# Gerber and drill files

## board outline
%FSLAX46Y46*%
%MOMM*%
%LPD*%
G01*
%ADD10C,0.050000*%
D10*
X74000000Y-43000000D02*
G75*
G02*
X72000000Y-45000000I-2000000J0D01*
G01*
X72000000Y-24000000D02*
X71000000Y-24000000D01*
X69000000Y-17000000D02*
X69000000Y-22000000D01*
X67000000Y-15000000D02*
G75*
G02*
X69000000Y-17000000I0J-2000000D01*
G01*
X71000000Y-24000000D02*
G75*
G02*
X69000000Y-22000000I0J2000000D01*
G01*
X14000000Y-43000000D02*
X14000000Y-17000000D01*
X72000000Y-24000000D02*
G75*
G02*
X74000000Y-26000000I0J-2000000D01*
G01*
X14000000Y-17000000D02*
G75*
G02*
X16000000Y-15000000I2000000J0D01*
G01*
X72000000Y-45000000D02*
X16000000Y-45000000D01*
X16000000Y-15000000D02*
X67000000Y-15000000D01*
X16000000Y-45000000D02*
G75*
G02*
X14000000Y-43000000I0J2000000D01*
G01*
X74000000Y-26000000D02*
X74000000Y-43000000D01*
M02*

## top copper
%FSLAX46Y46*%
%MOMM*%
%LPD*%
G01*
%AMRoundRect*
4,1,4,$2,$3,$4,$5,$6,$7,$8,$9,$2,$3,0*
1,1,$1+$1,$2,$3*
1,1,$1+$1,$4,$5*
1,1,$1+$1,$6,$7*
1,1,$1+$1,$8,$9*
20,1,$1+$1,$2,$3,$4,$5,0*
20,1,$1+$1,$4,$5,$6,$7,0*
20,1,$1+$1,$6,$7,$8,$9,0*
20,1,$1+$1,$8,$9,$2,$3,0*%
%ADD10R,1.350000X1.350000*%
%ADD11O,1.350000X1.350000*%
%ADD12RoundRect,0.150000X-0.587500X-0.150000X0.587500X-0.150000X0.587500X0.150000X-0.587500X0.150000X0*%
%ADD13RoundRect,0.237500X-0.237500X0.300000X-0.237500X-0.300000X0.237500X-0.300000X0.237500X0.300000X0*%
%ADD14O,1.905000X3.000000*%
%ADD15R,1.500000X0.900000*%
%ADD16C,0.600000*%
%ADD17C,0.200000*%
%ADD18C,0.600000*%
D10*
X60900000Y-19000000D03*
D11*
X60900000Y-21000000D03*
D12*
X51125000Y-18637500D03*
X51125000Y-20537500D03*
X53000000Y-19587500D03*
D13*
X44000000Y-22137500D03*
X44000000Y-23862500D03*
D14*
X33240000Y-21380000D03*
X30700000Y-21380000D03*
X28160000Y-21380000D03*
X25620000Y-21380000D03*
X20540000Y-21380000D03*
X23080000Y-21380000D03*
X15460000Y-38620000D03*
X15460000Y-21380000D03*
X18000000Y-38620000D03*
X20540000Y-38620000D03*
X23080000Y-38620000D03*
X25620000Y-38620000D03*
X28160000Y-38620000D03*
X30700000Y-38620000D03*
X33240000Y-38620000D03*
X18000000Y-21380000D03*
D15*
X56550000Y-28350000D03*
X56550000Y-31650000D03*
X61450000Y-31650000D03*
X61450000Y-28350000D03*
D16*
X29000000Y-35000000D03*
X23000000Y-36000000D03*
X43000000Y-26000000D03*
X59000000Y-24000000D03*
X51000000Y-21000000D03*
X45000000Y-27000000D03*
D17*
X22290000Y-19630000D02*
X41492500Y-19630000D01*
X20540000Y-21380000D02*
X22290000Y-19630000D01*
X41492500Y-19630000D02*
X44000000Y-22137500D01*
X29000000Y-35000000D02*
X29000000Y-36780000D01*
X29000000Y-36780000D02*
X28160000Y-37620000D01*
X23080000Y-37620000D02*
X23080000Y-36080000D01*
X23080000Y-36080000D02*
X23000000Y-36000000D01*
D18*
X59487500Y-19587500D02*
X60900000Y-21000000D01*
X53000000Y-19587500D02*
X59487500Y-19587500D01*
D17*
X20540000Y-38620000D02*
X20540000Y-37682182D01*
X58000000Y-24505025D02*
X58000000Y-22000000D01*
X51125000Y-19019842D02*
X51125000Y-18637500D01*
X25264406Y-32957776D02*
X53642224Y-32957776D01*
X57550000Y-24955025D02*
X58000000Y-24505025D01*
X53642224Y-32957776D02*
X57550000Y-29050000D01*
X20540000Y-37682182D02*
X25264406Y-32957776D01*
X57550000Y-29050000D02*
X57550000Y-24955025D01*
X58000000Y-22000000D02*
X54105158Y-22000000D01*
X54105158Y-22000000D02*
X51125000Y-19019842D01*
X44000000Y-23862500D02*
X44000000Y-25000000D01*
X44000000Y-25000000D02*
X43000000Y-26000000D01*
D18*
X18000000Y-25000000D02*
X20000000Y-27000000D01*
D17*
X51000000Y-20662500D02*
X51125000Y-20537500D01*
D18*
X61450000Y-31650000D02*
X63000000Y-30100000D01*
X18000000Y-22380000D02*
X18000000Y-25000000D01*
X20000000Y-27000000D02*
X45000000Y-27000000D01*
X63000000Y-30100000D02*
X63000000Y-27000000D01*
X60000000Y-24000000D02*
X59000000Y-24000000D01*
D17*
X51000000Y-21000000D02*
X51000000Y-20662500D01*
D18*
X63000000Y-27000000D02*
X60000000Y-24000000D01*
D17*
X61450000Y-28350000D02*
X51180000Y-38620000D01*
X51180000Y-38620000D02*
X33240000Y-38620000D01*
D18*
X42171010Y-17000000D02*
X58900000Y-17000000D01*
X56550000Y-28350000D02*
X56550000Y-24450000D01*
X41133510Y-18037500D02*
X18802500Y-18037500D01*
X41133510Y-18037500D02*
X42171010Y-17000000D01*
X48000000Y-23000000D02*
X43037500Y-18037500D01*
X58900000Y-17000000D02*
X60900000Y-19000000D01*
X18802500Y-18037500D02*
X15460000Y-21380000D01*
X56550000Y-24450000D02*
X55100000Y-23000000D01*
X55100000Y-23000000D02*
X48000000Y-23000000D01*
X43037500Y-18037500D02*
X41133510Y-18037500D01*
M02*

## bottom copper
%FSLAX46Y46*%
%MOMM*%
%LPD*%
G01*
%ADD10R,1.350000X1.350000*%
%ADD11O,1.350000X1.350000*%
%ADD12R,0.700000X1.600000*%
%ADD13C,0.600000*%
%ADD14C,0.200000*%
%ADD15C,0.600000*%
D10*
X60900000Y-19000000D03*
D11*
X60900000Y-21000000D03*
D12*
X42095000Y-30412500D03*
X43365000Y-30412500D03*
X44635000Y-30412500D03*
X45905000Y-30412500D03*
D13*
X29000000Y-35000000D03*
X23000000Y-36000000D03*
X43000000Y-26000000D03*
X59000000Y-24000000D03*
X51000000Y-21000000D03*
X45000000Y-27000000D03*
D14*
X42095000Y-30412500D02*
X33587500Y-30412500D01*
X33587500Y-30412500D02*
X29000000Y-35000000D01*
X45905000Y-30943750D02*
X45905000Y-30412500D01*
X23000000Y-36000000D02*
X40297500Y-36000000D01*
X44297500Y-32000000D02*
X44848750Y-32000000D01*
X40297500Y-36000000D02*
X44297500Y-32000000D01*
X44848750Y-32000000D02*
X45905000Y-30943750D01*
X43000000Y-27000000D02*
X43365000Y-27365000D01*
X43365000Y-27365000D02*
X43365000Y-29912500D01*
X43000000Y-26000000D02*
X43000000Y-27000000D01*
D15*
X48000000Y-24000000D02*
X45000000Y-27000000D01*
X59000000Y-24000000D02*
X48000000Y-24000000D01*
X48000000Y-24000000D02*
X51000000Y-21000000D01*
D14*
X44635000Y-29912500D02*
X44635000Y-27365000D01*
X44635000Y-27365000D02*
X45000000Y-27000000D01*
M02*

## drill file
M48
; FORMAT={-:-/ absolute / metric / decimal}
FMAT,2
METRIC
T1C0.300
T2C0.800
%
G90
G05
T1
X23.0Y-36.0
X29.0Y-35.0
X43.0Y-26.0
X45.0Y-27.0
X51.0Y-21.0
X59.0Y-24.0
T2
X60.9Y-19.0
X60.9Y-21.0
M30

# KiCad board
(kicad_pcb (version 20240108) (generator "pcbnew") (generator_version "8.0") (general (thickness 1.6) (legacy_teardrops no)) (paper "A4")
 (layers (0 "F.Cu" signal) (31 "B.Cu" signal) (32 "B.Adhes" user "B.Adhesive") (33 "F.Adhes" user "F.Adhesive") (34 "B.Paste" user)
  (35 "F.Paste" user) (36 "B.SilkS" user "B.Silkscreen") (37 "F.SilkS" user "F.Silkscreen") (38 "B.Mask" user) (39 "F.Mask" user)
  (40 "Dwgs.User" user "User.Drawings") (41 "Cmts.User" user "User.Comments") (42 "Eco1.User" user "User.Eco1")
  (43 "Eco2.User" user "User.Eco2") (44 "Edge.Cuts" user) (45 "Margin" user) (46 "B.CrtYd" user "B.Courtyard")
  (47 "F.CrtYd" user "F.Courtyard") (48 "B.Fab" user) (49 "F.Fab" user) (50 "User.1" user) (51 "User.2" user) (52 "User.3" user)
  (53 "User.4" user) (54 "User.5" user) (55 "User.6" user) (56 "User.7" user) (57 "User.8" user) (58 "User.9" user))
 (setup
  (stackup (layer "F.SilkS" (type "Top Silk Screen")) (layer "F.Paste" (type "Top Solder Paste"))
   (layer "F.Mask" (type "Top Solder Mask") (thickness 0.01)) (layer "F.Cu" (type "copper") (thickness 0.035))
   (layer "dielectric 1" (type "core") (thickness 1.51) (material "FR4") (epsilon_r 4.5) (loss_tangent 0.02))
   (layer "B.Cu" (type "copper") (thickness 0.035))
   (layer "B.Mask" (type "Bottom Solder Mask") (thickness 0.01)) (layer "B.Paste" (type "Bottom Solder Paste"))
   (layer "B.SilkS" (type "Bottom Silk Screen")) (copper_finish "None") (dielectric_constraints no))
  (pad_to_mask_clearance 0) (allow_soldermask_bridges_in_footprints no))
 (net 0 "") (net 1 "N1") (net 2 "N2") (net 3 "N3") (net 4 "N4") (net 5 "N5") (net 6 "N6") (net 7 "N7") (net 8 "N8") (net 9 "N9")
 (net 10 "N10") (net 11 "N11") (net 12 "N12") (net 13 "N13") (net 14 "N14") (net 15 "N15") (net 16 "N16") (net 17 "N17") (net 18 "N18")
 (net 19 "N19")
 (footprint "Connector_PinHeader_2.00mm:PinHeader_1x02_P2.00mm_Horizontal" (layer "F.Cu") (at 60.9 19)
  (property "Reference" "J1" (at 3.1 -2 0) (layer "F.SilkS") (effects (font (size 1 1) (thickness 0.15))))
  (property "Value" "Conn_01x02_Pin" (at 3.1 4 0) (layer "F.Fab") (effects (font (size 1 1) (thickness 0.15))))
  (pad "1" thru_hole rect (at 0 0) (size 1.35 1.35) (drill 0.8) (layers "*.Cu" "*.Mask") (remove_unused_layers no) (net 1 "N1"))
  (pad "2" thru_hole oval (at 0 2) (size 1.35 1.35) (drill 0.8) (layers "*.Cu" "*.Mask") (remove_unused_layers no) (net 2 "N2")))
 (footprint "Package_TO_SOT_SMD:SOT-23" (layer "F.Cu") (at 52.0625 19.5875)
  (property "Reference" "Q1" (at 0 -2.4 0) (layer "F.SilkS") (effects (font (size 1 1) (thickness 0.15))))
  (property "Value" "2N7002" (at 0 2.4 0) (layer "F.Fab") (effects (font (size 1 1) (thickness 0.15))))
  (pad "1" smd roundrect (at -0.9375 -0.95) (size 1.475 0.6) (layers "F.Cu" "F.Paste" "F.Mask") (roundrect_rratio 0.25) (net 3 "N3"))
  (pad "2" smd roundrect (at -0.9375 0.95) (size 1.475 0.6) (layers "F.Cu" "F.Paste" "F.Mask") (roundrect_rratio 0.25) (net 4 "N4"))
  (pad "3" smd roundrect (at 0.9375 0) (size 1.475 0.6) (layers "F.Cu" "F.Paste" "F.Mask") (roundrect_rratio 0.25) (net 2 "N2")))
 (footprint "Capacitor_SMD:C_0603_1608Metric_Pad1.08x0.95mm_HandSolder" (layer "F.Cu") (at 44 23 -90)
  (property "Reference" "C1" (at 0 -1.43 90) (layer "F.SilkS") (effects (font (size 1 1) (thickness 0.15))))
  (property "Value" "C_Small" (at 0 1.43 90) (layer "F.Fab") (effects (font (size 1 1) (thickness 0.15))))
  (pad "1" smd roundrect (at -0.8625 0 270) (size 1.075 0.95) (layers "F.Cu" "F.Paste" "F.Mask") (roundrect_rratio 0.25) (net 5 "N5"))
  (pad "2" smd roundrect (at 0.8625 0 270) (size 1.075 0.95) (layers "F.Cu" "F.Paste" "F.Mask") (roundrect_rratio 0.25) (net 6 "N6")))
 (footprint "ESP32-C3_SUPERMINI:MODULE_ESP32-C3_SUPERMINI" (layer "F.Cu") (at 25.36 30 90)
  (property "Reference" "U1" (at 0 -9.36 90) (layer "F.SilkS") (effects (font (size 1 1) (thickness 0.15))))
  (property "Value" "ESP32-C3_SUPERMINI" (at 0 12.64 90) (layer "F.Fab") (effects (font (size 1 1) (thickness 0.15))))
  (pad "0" connect oval (at 8.62 7.88 90) (size 3 1.905) (layers "F.Cu" "F.Mask") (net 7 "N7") (solder_mask_margin 0.102))
  (pad "1" connect oval (at 8.62 5.34 90) (size 3 1.905) (layers "F.Cu" "F.Mask") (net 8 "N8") (solder_mask_margin 0.102))
  (pad "2" connect oval (at 8.62 2.8 90) (size 3 1.905) (layers "F.Cu" "F.Mask") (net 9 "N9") (solder_mask_margin 0.102))
  (pad "3" connect oval (at 8.62 0.26 90) (size 3 1.905) (layers "F.Cu" "F.Mask") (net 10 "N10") (solder_mask_margin 0.102))
  (pad "3.3" connect oval (at 8.62 -4.82 90) (size 3 1.905) (layers "F.Cu" "F.Mask") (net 5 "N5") (solder_mask_margin 0.102))
  (pad "4" connect oval (at 8.62 -2.28 90) (size 3 1.905) (layers "F.Cu" "F.Mask") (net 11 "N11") (solder_mask_margin 0.102))
  (pad "5" connect oval (at -8.62 -9.9 90) (size 3 1.905) (layers "F.Cu" "F.Mask") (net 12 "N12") (solder_mask_margin 0.102))
  (pad "5V" connect oval (at 8.62 -9.9 90) (size 3 1.905) (layers "F.Cu" "F.Mask") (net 1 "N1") (solder_mask_margin 0.102))
  (pad "6" connect oval (at -8.62 -7.36 90) (size 3 1.905) (layers "F.Cu" "F.Mask") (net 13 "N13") (solder_mask_margin 0.102))
  (pad "7" connect oval (at -8.62 -4.82 90) (size 3 1.905) (layers "F.Cu" "F.Mask") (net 3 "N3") (solder_mask_margin 0.102))
  (pad "8" connect oval (at -8.62 -2.28 90) (size 3 1.905) (layers "F.Cu" "F.Mask") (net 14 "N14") (solder_mask_margin 0.102))
  (pad "9" connect oval (at -8.62 0.26 90) (size 3 1.905) (layers "F.Cu" "F.Mask") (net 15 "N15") (solder_mask_margin 0.102))
  (pad "10" connect oval (at -8.62 2.8 90) (size 3 1.905) (layers "F.Cu" "F.Mask") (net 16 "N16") (solder_mask_margin 0.102))
  (pad "20" connect oval (at -8.62 5.34 90) (size 3 1.905) (layers "F.Cu" "F.Mask") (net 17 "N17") (solder_mask_margin 0.102))
  (pad "21" connect oval (at -8.62 7.88 90) (size 3 1.905) (layers "F.Cu" "F.Mask") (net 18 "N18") (solder_mask_margin 0.102))
  (pad "G" connect oval (at 8.62 -7.36 90) (size 3 1.905) (layers "F.Cu" "F.Mask") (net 4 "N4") (solder_mask_margin 0.102)))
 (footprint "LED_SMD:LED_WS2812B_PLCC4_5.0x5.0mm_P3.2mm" (layer "F.Cu") (at 59 30)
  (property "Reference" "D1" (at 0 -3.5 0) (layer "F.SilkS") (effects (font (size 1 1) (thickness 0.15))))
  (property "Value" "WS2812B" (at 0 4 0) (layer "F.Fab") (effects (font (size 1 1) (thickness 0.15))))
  (pad "1" smd rect (at -2.45 -1.65) (size 1.5 0.9) (layers "F.Cu" "F.Paste" "F.Mask") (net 1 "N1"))
  (pad "2" smd rect (at -2.45 1.65) (size 1.5 0.9) (layers "F.Cu" "F.Paste" "F.Mask") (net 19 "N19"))
  (pad "3" smd rect (at 2.45 1.65) (size 1.5 0.9) (layers "F.Cu" "F.Paste" "F.Mask") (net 4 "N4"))
  (pad "4" smd rect (at 2.45 -1.65) (size 1.5 0.9) (layers "F.Cu" "F.Paste" "F.Mask") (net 18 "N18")))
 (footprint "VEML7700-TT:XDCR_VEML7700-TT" (layer "B.Cu") (at 44 31.3125 -90)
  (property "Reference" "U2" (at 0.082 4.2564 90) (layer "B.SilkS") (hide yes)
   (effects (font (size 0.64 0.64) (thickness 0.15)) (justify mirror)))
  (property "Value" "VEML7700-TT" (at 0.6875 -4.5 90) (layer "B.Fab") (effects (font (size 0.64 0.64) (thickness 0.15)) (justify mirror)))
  (pad "1" smd rect (at -0.9 1.905 270) (size 1.6 0.7) (layers "B.Cu" "B.Paste" "B.Mask") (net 16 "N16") (solder_mask_margin 0.102))
  (pad "2" smd rect (at -0.9 0.635 270) (size 1.6 0.7) (layers "B.Cu" "B.Paste" "B.Mask") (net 6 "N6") (solder_mask_margin 0.102))
  (pad "3" smd rect (at -0.9 -0.635 270) (size 1.6 0.7) (layers "B.Cu" "B.Paste" "B.Mask") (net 4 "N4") (solder_mask_margin 0.102))
  (pad "4" smd rect (at -0.9 -1.905 270) (size 1.6 0.7) (layers "B.Cu" "B.Paste" "B.Mask") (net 14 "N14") (solder_mask_margin 0.102)))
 (gr_arc (start 74 43) (mid 73.414214 44.414214) (end 72 45) (stroke (width 0.05) (type default)) (layer "Edge.Cuts"))
 (gr_line (start 72 24) (end 71 24) (stroke (width 0.05) (type default)) (layer "Edge.Cuts"))
 (gr_line (start 69 17) (end 69 22) (stroke (width 0.05) (type default)) (layer "Edge.Cuts"))
 (gr_arc (start 67 15) (mid 68.414214 15.585786) (end 69 17) (stroke (width 0.05) (type default)) (layer "Edge.Cuts"))
 (gr_arc (start 71 24) (mid 69.585786 23.414214) (end 69 22) (stroke (width 0.05) (type default)) (layer "Edge.Cuts"))
 (gr_line (start 14 43) (end 14 17) (stroke (width 0.05) (type default)) (layer "Edge.Cuts"))
 (gr_arc (start 72 24) (mid 73.414214 24.585786) (end 74 26) (stroke (width 0.05) (type default)) (layer "Edge.Cuts"))
 (gr_arc (start 14 17) (mid 14.585786 15.585786) (end 16 15) (stroke (width 0.05) (type default)) (layer "Edge.Cuts"))
 (gr_line (start 72 45) (end 16 45) (stroke (width 0.05) (type default)) (layer "Edge.Cuts"))
 (gr_line (start 16 15) (end 67 15) (stroke (width 0.05) (type default)) (layer "Edge.Cuts"))
 (gr_arc (start 16 45) (mid 14.585786 44.414214) (end 14 43) (stroke (width 0.05) (type default)) (layer "Edge.Cuts"))
 (gr_line (start 74 26) (end 74 43) (stroke (width 0.05) (type default)) (layer "Edge.Cuts"))
 (segment (start 22.29 19.63) (end 41.4925 19.63) (width 0.2) (layer "F.Cu") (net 5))
 (segment (start 20.54 21.38) (end 22.29 19.63) (width 0.2) (layer "F.Cu") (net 5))
 (segment (start 41.4925 19.63) (end 44 22.1375) (width 0.2) (layer "F.Cu") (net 5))
 (segment (start 29 35) (end 29 36.78) (width 0.2) (layer "F.Cu") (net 16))
 (segment (start 29 36.78) (end 28.16 37.62) (width 0.2) (layer "F.Cu") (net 16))
 (via (at 29 35) (size 0.6) (drill 0.3) (layers "F.Cu" "B.Cu") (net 16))
 (segment (start 42.095 30.4125) (end 33.5875 30.4125) (width 0.2) (layer "B.Cu") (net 16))
 (segment (start 33.5875 30.4125) (end 29 35) (width 0.2) (layer "B.Cu") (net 16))
 (segment (start 23.08 37.62) (end 23.08 36.08) (width 0.2) (layer "F.Cu") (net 14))
 (segment (start 23.08 36.08) (end 23 36) (width 0.2) (layer "F.Cu") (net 14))
 (via (at 23 36) (size 0.6) (drill 0.3) (layers "F.Cu" "B.Cu") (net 14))
 (segment (start 45.905 30.94375) (end 45.905 30.4125) (width 0.2) (layer "B.Cu") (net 14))
 (segment (start 23 36) (end 40.2975 36) (width 0.2) (layer "B.Cu") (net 14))
 (segment (start 44.2975 32) (end 44.84875 32) (width 0.2) (layer "B.Cu") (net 14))
 (segment (start 40.2975 36) (end 44.2975 32) (width 0.2) (layer "B.Cu") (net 14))
 (segment (start 44.84875 32) (end 45.905 30.94375) (width 0.2) (layer "B.Cu") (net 14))
 (segment (start 59.4875 19.5875) (end 60.9 21) (width 0.6) (layer "F.Cu") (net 2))
 (segment (start 53 19.5875) (end 59.4875 19.5875) (width 0.6) (layer "F.Cu") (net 2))
 (segment (start 20.54 38.62) (end 20.54 37.682182) (width 0.2) (layer "F.Cu") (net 3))
 (segment (start 58 24.505025) (end 58 22) (width 0.2) (layer "F.Cu") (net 3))
 (segment (start 51.125 19.019842) (end 51.125 18.6375) (width 0.2) (layer "F.Cu") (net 3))
 (segment (start 25.264406 32.957776) (end 53.642224 32.957776) (width 0.2) (layer "F.Cu") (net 3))
 (segment (start 57.55 24.955025) (end 58 24.505025) (width 0.2) (layer "F.Cu") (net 3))
 (segment (start 53.642224 32.957776) (end 57.55 29.05) (width 0.2) (layer "F.Cu") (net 3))
 (segment (start 20.54 37.682182) (end 25.264406 32.957776) (width 0.2) (layer "F.Cu") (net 3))
 (segment (start 57.55 29.05) (end 57.55 24.955025) (width 0.2) (layer "F.Cu") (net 3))
 (segment (start 58 22) (end 54.105158 22) (width 0.2) (layer "F.Cu") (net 3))
 (segment (start 54.105158 22) (end 51.125 19.019842) (width 0.2) (layer "F.Cu") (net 3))
 (segment (start 44 23.8625) (end 44 25) (width 0.2) (layer "F.Cu") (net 6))
 (segment (start 44 25) (end 43 26) (width 0.2) (layer "F.Cu") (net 6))
 (via (at 43 26) (size 0.6) (drill 0.3) (layers "F.Cu" "B.Cu") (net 6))
 (segment (start 43 27) (end 43.365 27.365) (width 0.2) (layer "B.Cu") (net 6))
 (segment (start 43.365 27.365) (end 43.365 29.9125) (width 0.2) (layer "B.Cu") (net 6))
 (segment (start 43 26) (end 43 27) (width 0.2) (layer "B.Cu") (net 6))
 (segment (start 18 25) (end 20 27) (width 0.6) (layer "F.Cu") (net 4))
 (segment (start 51 20.6625) (end 51.125 20.5375) (width 0.2) (layer "F.Cu") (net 4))
 (segment (start 61.45 31.65) (end 63 30.1) (width 0.6) (layer "F.Cu") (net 4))
 (segment (start 18 22.38) (end 18 25) (width 0.6) (layer "F.Cu") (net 4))
 (segment (start 20 27) (end 45 27) (width 0.6) (layer "F.Cu") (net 4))
 (segment (start 63 30.1) (end 63 27) (width 0.6) (layer "F.Cu") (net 4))
 (segment (start 60 24) (end 59 24) (width 0.6) (layer "F.Cu") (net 4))
 (segment (start 51 21) (end 51 20.6625) (width 0.2) (layer "F.Cu") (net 4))
 (segment (start 63 27) (end 60 24) (width 0.6) (layer "F.Cu") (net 4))
 (via (at 59 24) (size 0.6) (drill 0.3) (layers "F.Cu" "B.Cu") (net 4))
 (via (at 51 21) (size 0.6) (drill 0.3) (layers "F.Cu" "B.Cu") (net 4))
 (via (at 45 27) (size 0.6) (drill 0.3) (layers "F.Cu" "B.Cu") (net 4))
 (segment (start 48 24) (end 45 27) (width 0.6) (layer "B.Cu") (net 4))
 (segment (start 59 24) (end 48 24) (width 0.6) (layer "B.Cu") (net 4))
 (segment (start 48 24) (end 51 21) (width 0.6) (layer "B.Cu") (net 4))
 (segment (start 44.635 29.9125) (end 44.635 27.365) (width 0.2) (layer "B.Cu") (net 4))
 (segment (start 44.635 27.365) (end 45 27) (width 0.2) (layer "B.Cu") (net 4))
 (segment (start 61.45 28.35) (end 51.18 38.62) (width 0.2) (layer "F.Cu") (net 18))
 (segment (start 51.18 38.62) (end 33.24 38.62) (width 0.2) (layer "F.Cu") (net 18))
 (segment (start 42.17101 17) (end 58.9 17) (width 0.6) (layer "F.Cu") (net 1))
 (segment (start 56.55 28.35) (end 56.55 24.45) (width 0.6) (layer "F.Cu") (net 1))
 (segment (start 41.13351 18.0375) (end 18.8025 18.0375) (width 0.6) (layer "F.Cu") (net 1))
 (segment (start 41.13351 18.0375) (end 42.17101 17) (width 0.6) (layer "F.Cu") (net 1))
 (segment (start 48 23) (end 43.0375 18.0375) (width 0.6) (layer "F.Cu") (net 1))
 (segment (start 58.9 17) (end 60.9 19) (width 0.6) (layer "F.Cu") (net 1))
 (segment (start 18.8025 18.0375) (end 15.46 21.38) (width 0.6) (layer "F.Cu") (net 1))
 (segment (start 56.55 24.45) (end 55.1 23) (width 0.6) (layer "F.Cu") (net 1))
 (segment (start 55.1 23) (end 48 23) (width 0.6) (layer "F.Cu") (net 1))
 (segment (start 43.0375 18.0375) (end 41.13351 18.0375) (width 0.6) (layer "F.Cu") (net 1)))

